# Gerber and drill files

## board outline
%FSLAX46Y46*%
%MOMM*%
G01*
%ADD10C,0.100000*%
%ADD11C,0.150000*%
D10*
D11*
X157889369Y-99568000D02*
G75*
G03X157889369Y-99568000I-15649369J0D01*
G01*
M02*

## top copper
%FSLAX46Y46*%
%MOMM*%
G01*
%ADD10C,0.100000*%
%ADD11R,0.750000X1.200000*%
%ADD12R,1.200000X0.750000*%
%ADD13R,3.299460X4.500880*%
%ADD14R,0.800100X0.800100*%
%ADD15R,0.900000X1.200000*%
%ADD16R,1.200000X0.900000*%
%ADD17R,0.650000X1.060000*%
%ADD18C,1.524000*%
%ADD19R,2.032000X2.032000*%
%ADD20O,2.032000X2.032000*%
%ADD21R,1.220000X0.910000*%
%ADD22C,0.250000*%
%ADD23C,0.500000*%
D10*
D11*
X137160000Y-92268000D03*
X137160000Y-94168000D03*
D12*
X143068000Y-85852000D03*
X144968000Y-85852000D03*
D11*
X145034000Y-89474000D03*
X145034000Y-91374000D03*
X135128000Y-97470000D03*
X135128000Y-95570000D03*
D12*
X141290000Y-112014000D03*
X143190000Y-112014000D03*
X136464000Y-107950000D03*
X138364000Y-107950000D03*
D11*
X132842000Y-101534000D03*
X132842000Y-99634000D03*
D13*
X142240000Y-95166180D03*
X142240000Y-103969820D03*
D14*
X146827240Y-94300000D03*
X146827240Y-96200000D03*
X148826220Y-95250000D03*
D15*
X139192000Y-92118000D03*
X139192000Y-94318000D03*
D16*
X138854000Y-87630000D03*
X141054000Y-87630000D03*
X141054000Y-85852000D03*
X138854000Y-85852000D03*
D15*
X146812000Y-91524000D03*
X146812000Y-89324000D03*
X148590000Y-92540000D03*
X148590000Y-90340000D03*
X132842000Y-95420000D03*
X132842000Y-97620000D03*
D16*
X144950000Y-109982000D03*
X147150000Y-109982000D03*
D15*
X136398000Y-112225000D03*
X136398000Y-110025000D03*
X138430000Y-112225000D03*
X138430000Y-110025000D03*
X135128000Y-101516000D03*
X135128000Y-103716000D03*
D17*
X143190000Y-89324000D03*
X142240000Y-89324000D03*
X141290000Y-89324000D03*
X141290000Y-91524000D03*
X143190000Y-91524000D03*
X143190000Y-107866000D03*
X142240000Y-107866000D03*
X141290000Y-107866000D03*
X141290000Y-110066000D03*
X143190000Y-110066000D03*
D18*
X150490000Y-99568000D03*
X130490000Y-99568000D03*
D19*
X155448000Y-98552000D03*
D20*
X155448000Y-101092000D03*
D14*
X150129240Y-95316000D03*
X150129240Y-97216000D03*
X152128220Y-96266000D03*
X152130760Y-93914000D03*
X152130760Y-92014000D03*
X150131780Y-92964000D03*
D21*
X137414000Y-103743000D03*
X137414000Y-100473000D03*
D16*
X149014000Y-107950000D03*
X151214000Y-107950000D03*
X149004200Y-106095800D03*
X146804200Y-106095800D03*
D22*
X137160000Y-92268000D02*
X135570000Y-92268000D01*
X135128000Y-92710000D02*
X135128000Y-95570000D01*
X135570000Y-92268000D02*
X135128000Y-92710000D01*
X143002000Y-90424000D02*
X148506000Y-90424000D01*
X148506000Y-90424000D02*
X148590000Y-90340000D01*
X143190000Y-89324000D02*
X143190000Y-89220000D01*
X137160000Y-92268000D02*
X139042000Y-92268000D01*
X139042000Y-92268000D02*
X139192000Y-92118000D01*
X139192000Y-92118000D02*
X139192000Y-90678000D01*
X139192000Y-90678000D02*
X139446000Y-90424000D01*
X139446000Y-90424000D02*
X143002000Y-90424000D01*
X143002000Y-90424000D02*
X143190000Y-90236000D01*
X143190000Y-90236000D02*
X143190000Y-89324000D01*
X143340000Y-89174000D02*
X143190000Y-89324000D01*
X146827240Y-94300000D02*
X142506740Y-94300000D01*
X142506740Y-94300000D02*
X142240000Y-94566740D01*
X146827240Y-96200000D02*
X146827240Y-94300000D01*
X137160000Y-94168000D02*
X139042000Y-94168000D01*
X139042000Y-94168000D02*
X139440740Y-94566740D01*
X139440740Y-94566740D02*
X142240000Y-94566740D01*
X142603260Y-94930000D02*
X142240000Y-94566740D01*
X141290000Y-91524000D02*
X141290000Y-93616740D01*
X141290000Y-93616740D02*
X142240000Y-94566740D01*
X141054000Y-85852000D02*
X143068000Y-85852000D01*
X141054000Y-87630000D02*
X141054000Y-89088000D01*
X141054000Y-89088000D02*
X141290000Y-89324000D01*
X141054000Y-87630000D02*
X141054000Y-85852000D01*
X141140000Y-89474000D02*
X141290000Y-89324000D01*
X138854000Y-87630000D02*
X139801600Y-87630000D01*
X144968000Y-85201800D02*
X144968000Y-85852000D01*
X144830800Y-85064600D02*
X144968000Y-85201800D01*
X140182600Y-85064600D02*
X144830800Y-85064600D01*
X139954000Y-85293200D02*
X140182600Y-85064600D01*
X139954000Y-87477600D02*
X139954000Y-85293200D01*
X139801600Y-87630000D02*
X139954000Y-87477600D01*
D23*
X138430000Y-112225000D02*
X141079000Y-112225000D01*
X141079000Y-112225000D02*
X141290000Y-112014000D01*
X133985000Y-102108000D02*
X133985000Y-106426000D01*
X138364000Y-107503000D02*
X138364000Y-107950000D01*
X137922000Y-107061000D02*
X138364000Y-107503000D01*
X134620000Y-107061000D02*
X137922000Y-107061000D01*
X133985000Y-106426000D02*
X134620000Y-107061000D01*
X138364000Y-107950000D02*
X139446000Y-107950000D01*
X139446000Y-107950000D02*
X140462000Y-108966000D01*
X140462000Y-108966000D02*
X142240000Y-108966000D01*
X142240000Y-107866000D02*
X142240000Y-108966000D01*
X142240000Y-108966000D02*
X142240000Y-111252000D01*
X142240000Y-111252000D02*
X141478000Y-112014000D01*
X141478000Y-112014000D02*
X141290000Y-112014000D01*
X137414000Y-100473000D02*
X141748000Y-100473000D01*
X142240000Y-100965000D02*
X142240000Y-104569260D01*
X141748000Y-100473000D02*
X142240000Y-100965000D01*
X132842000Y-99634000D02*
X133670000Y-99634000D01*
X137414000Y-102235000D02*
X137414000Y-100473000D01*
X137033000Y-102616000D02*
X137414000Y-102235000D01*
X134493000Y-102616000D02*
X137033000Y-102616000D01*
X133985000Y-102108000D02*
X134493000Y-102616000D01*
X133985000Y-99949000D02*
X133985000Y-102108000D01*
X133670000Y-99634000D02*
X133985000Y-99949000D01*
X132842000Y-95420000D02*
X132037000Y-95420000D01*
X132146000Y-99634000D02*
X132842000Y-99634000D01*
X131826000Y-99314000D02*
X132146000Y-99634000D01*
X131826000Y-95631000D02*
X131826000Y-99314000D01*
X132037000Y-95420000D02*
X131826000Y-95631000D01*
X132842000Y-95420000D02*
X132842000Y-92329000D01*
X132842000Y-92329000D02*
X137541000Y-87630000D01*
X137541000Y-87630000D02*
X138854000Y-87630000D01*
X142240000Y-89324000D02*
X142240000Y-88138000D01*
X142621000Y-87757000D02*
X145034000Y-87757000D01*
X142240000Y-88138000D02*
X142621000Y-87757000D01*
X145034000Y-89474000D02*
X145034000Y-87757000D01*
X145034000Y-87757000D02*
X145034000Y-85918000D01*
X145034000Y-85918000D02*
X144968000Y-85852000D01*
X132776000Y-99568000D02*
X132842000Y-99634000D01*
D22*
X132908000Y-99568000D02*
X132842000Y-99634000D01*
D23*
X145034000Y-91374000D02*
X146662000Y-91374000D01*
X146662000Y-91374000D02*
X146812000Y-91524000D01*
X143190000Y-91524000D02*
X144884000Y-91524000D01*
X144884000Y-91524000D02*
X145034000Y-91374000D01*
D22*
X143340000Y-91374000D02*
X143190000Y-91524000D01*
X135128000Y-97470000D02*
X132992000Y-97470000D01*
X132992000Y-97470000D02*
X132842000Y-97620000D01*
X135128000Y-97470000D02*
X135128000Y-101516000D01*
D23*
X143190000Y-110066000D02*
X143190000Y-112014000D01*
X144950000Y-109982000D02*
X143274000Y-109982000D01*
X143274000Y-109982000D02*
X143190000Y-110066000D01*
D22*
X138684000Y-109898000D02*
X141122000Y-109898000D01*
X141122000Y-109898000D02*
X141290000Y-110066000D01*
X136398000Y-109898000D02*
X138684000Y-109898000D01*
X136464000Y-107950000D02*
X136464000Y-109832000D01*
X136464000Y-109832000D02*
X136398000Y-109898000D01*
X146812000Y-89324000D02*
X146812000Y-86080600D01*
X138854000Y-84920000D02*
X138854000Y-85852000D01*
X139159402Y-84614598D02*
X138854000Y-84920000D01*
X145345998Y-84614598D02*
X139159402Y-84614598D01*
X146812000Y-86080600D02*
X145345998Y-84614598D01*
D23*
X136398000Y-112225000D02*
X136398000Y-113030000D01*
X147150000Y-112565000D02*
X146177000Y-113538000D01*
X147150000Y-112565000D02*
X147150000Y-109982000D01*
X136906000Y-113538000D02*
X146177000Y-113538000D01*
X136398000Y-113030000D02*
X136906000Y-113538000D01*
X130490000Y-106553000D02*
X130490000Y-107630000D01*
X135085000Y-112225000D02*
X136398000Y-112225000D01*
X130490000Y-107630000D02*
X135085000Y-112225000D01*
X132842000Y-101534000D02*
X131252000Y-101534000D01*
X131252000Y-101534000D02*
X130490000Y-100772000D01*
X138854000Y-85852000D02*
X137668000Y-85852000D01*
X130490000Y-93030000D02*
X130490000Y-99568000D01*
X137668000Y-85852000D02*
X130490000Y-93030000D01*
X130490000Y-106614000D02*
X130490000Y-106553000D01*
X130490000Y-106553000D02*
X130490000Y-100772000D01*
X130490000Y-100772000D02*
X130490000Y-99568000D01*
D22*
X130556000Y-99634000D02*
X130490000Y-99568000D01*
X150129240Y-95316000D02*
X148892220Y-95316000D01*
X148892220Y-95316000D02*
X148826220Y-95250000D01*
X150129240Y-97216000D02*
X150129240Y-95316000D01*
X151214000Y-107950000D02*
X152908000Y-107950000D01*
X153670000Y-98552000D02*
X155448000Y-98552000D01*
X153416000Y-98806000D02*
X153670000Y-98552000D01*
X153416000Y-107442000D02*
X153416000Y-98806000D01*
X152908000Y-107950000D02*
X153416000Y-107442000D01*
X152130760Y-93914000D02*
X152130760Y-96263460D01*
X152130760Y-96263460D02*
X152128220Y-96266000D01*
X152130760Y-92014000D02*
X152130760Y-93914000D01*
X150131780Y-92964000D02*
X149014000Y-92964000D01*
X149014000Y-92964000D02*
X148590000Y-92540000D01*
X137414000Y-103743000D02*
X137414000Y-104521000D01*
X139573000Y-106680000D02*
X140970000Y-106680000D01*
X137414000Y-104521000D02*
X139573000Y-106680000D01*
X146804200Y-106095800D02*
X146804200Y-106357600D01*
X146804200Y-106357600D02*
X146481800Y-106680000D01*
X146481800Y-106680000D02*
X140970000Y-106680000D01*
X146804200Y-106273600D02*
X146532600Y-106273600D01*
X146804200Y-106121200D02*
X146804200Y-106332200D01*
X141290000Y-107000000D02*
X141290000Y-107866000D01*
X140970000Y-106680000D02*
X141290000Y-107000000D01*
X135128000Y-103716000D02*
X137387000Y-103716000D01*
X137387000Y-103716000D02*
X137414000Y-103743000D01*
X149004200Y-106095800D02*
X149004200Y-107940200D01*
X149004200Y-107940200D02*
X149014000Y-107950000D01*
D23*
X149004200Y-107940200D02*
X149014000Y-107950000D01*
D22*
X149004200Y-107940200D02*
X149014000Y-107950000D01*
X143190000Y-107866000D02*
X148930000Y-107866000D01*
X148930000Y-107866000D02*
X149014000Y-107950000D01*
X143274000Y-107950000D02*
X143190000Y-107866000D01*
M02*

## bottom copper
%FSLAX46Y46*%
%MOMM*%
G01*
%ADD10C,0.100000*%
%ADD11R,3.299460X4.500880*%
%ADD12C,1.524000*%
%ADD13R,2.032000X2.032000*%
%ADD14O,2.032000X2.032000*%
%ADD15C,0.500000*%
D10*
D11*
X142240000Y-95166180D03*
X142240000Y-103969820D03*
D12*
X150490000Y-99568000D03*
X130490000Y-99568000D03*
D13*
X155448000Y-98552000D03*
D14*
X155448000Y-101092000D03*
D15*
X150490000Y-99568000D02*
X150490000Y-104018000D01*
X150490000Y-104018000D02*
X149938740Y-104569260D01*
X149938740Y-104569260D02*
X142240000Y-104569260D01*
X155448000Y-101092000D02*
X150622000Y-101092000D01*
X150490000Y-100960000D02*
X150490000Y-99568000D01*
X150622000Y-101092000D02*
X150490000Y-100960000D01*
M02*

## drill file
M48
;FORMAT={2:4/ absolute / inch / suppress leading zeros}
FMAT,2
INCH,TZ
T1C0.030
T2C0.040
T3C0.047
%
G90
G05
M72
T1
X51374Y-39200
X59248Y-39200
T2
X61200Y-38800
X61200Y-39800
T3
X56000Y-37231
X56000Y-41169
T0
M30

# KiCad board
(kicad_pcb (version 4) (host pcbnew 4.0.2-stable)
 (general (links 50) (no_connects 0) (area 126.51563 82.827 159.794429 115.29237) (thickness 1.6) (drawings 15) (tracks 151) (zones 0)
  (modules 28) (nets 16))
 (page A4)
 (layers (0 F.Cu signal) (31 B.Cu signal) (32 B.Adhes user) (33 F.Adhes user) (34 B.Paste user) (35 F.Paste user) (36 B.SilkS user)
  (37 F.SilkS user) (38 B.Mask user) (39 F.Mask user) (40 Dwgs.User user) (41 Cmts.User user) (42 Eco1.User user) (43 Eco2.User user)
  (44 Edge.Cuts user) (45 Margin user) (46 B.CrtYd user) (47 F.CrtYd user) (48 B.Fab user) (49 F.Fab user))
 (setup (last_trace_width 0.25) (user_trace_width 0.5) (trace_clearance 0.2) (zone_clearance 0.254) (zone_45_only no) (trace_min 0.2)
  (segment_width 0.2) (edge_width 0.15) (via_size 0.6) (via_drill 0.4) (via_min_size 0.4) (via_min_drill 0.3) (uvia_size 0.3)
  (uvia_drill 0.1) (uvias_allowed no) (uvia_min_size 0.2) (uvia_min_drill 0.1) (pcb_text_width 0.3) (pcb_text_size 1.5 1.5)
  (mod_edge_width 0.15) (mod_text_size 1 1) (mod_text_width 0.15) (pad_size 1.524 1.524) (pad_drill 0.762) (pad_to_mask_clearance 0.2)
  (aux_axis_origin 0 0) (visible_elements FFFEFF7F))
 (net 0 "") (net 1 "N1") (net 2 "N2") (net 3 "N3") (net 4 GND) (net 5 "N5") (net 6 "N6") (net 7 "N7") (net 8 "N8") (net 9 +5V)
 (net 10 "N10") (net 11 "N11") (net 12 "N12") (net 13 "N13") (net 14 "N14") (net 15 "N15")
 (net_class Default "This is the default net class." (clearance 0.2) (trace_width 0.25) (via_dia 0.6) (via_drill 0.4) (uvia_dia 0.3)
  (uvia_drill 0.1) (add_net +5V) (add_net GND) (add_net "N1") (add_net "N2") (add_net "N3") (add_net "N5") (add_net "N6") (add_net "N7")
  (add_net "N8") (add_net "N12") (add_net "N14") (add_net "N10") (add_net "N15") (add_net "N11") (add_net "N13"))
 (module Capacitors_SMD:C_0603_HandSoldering (layer F.Cu) (at 137.16 93.218 270)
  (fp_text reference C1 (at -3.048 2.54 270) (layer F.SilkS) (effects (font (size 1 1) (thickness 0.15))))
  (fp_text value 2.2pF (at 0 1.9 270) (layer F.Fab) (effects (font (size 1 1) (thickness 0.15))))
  (pad 1 smd rect (at -0.95 0 270) (size 1.2 0.75) (layers F.Cu F.Paste F.Mask) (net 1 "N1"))
  (pad 2 smd rect (at 0.95 0 270) (size 1.2 0.75) (layers F.Cu F.Paste F.Mask) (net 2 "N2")))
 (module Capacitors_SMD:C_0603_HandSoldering (layer F.Cu) (at 144.018 85.852)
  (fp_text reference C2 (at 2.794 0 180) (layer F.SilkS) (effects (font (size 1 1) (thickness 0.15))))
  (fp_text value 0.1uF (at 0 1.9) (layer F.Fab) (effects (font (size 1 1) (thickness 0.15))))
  (pad 1 smd rect (at -0.95 0) (size 1.2 0.75) (layers F.Cu F.Paste F.Mask) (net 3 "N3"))
  (pad 2 smd rect (at 0.95 0) (size 1.2 0.75) (layers F.Cu F.Paste F.Mask) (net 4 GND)))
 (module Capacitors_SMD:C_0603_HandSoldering (layer F.Cu) (at 145.034 90.424 270)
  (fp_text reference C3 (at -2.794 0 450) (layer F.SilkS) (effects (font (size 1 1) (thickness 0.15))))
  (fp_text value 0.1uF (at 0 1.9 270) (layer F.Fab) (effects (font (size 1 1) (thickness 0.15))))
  (pad 1 smd rect (at -0.95 0 270) (size 1.2 0.75) (layers F.Cu F.Paste F.Mask) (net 4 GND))
  (pad 2 smd rect (at 0.95 0 270) (size 1.2 0.75) (layers F.Cu F.Paste F.Mask) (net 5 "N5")))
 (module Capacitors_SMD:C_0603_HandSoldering (layer F.Cu) (at 135.128 96.52 90)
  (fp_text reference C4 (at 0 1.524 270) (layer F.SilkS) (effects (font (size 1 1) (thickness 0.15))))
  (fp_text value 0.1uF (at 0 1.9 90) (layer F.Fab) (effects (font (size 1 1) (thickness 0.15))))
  (pad 1 smd rect (at -0.95 0 90) (size 1.2 0.75) (layers F.Cu F.Paste F.Mask) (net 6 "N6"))
  (pad 2 smd rect (at 0.95 0 90) (size 1.2 0.75) (layers F.Cu F.Paste F.Mask) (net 1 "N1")))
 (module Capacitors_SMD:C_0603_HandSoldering (layer F.Cu) (at 142.24 112.014)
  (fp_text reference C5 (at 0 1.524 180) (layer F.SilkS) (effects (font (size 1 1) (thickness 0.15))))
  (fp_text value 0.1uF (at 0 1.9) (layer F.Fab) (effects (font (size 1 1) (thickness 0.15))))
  (pad 1 smd rect (at -0.95 0) (size 1.2 0.75) (layers F.Cu F.Paste F.Mask) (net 4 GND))
  (pad 2 smd rect (at 0.95 0) (size 1.2 0.75) (layers F.Cu F.Paste F.Mask) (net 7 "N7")))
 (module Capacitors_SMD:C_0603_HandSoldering (layer F.Cu) (at 137.414 107.95)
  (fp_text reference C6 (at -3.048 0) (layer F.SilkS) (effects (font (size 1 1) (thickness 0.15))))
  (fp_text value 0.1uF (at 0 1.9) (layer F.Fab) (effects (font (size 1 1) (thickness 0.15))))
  (pad 1 smd rect (at -0.95 0) (size 1.2 0.75) (layers F.Cu F.Paste F.Mask) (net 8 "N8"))
  (pad 2 smd rect (at 0.95 0) (size 1.2 0.75) (layers F.Cu F.Paste F.Mask) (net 4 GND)))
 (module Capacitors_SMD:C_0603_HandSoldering (layer F.Cu) (at 132.842 100.584 90)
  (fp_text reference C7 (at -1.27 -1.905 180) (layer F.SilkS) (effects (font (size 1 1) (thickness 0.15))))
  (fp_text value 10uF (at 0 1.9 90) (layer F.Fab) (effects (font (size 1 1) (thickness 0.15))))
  (pad 1 smd rect (at -0.95 0 90) (size 1.2 0.75) (layers F.Cu F.Paste F.Mask) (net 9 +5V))
  (pad 2 smd rect (at 0.95 0 90) (size 1.2 0.75) (layers F.Cu F.Paste F.Mask) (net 4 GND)))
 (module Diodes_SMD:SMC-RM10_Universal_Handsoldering (layer F.Cu) (at 142.24 99.568 270)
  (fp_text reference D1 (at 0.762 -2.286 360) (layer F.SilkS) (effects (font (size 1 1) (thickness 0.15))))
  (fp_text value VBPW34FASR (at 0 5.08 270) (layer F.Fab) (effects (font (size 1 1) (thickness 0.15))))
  (pad 1 thru_hole rect (at -5.00126 0 270) (size 4.50088 3.29946) (drill 1.19888 (offset 0.59944 0)) (layers *.Cu *.Mask F.SilkS)
   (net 2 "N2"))
  (pad 2 thru_hole rect (at 5.00126 0 90) (size 4.50088 3.29946) (drill 1.19888 (offset 0.59944 0)) (layers *.Cu *.Mask F.SilkS) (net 4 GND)))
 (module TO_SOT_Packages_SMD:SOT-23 (layer F.Cu) (at 147.828 95.25 270)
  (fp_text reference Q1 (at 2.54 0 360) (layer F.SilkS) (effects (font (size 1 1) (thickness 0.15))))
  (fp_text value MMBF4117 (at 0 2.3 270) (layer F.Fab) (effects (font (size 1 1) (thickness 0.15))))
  (pad 1 smd rect (at -0.95 1.00076 270) (size 0.8001 0.8001) (layers F.Cu F.Paste F.Mask) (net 2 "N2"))
  (pad 2 smd rect (at 0.95 1.00076 270) (size 0.8001 0.8001) (layers F.Cu F.Paste F.Mask) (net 2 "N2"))
  (pad 3 smd rect (at 0 -0.99822 270) (size 0.8001 0.8001) (layers F.Cu F.Paste F.Mask) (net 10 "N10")))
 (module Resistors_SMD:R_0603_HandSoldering (layer F.Cu) (at 139.192 93.218 270)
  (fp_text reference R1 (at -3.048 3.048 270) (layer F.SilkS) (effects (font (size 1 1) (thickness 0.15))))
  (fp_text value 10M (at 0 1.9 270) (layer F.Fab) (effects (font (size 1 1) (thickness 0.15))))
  (pad 1 smd rect (at -1.1 0 270) (size 1.2 0.9) (layers F.Cu F.Paste F.Mask) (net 1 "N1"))
  (pad 2 smd rect (at 1.1 0 270) (size 1.2 0.9) (layers F.Cu F.Paste F.Mask) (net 2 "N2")))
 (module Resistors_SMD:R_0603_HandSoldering (layer F.Cu) (at 139.954 87.63)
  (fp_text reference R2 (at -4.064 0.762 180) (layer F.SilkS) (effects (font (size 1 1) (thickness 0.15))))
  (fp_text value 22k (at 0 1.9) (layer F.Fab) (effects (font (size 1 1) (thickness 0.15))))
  (pad 1 smd rect (at -1.1 0) (size 1.2 0.9) (layers F.Cu F.Paste F.Mask) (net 4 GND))
  (pad 2 smd rect (at 1.1 0) (size 1.2 0.9) (layers F.Cu F.Paste F.Mask) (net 3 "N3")))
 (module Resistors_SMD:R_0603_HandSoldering (layer F.Cu) (at 139.954 85.852 180)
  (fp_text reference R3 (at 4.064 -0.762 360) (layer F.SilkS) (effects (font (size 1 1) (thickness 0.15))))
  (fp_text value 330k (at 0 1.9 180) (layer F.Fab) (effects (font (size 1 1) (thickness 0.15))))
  (pad 1 smd rect (at -1.1 0 180) (size 1.2 0.9) (layers F.Cu F.Paste F.Mask) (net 3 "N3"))
  (pad 2 smd rect (at 1.1 0 180) (size 1.2 0.9) (layers F.Cu F.Paste F.Mask) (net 9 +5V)))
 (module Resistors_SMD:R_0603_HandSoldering (layer F.Cu) (at 146.812 90.424 90)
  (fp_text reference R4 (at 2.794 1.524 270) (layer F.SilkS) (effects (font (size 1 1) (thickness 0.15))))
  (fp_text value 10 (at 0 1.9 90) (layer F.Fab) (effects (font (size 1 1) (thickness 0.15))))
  (pad 1 smd rect (at -1.1 0 90) (size 1.2 0.9) (layers F.Cu F.Paste F.Mask) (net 5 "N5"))
  (pad 2 smd rect (at 1.1 0 90) (size 1.2 0.9) (layers F.Cu F.Paste F.Mask) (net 9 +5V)))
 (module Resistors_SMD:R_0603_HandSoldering (layer F.Cu) (at 148.59 91.44 90)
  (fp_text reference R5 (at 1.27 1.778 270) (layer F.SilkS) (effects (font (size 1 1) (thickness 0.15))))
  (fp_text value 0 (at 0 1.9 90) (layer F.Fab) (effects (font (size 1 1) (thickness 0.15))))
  (pad 1 smd rect (at -1.1 0 90) (size 1.2 0.9) (layers F.Cu F.Paste F.Mask) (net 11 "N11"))
  (pad 2 smd rect (at 1.1 0 90) (size 1.2 0.9) (layers F.Cu F.Paste F.Mask) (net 1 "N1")))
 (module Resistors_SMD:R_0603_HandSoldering (layer F.Cu) (at 132.842 96.52 270)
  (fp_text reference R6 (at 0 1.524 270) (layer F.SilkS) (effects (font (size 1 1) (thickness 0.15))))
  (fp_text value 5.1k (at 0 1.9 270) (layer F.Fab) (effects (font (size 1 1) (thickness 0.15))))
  (pad 1 smd rect (at -1.1 0 270) (size 1.2 0.9) (layers F.Cu F.Paste F.Mask) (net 4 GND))
  (pad 2 smd rect (at 1.1 0 270) (size 1.2 0.9) (layers F.Cu F.Paste F.Mask) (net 6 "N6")))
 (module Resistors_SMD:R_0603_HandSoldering (layer F.Cu) (at 146.05 109.982)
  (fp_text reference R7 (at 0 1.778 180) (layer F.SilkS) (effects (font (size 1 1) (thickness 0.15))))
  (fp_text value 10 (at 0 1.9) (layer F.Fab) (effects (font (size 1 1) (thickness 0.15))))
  (pad 1 smd rect (at -1.1 0) (size 1.2 0.9) (layers F.Cu F.Paste F.Mask) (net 7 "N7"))
  (pad 2 smd rect (at 1.1 0) (size 1.2 0.9) (layers F.Cu F.Paste F.Mask) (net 9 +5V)))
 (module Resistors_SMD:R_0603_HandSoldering (layer F.Cu) (at 136.398 111.125 90)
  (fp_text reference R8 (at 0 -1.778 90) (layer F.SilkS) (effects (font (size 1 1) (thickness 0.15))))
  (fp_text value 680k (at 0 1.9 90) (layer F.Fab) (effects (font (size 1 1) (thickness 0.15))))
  (pad 1 smd rect (at -1.1 0 90) (size 1.2 0.9) (layers F.Cu F.Paste F.Mask) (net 9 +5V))
  (pad 2 smd rect (at 1.1 0 90) (size 1.2 0.9) (layers F.Cu F.Paste F.Mask) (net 8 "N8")))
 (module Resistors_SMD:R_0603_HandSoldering (layer F.Cu) (at 138.43 111.125 90)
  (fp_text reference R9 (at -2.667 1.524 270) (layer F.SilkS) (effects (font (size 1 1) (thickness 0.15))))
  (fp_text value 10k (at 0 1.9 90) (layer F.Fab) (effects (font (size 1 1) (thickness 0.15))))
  (pad 1 smd rect (at -1.1 0 90) (size 1.2 0.9) (layers F.Cu F.Paste F.Mask) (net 4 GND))
  (pad 2 smd rect (at 1.1 0 90) (size 1.2 0.9) (layers F.Cu F.Paste F.Mask) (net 8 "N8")))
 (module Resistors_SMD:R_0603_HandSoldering (layer F.Cu) (at 135.128 102.616 270)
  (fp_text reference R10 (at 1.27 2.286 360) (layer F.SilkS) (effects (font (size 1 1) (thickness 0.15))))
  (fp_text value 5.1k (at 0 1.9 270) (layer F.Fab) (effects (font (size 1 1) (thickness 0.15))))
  (pad 1 smd rect (at -1.1 0 270) (size 1.2 0.9) (layers F.Cu F.Paste F.Mask) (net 6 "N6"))
  (pad 2 smd rect (at 1.1 0 270) (size 1.2 0.9) (layers F.Cu F.Paste F.Mask) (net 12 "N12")))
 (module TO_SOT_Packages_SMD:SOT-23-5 (layer F.Cu) (at 142.24 90.424 270)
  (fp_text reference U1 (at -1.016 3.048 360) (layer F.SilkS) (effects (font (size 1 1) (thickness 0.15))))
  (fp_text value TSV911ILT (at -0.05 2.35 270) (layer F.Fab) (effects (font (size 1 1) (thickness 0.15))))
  (pad 1 smd rect (at -1.1 -0.95 270) (size 1.06 0.65) (layers F.Cu F.Paste F.Mask) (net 1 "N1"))
  (pad 2 smd rect (at -1.1 0 270) (size 1.06 0.65) (layers F.Cu F.Paste F.Mask) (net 4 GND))
  (pad 3 smd rect (at -1.1 0.95 270) (size 1.06 0.65) (layers F.Cu F.Paste F.Mask) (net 3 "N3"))
  (pad 4 smd rect (at 1.1 0.95 270) (size 1.06 0.65) (layers F.Cu F.Paste F.Mask) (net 2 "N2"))
  (pad 5 smd rect (at 1.1 -0.95 270) (size 1.06 0.65) (layers F.Cu F.Paste F.Mask) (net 5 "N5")))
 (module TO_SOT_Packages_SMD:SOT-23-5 (layer F.Cu) (at 142.24 108.966 270)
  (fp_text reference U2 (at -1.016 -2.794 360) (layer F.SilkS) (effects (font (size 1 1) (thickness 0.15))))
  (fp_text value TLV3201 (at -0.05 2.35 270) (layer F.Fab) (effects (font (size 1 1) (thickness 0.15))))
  (pad 1 smd rect (at -1.1 -0.95 270) (size 1.06 0.65) (layers F.Cu F.Paste F.Mask) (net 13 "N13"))
  (pad 2 smd rect (at -1.1 0 270) (size 1.06 0.65) (layers F.Cu F.Paste F.Mask) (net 4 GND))
  (pad 3 smd rect (at -1.1 0.95 270) (size 1.06 0.65) (layers F.Cu F.Paste F.Mask) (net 12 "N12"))
  (pad 4 smd rect (at 1.1 0.95 270) (size 1.06 0.65) (layers F.Cu F.Paste F.Mask) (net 8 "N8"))
  (pad 5 smd rect (at 1.1 -0.95 270) (size 1.06 0.65) (layers F.Cu F.Paste F.Mask) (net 7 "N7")))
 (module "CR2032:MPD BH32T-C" (layer B.Cu) (at 142.24 99.568 90)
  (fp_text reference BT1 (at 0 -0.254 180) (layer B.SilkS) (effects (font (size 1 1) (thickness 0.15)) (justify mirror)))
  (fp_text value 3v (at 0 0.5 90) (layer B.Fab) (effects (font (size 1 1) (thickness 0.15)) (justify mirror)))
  (pad 2 thru_hole circle (at 0 8.25 90) (size 1.524 1.524) (drill 0.762) (layers *.Cu *.Mask B.SilkS) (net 4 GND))
  (pad 1 thru_hole circle (at 0 -11.75 90) (size 1.524 1.524) (drill 0.762) (layers *.Cu *.Mask B.SilkS) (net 9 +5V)))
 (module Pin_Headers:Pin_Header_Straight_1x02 (layer F.Cu) (at 155.448 98.552)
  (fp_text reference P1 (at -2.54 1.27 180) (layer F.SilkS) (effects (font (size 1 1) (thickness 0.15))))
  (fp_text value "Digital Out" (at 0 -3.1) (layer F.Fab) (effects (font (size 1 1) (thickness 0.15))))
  (pad 1 thru_hole rect (at 0 0) (size 2.032 2.032) (drill 1.016) (layers *.Cu *.Mask F.SilkS) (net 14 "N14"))
  (pad 2 thru_hole oval (at 0 2.54) (size 2.032 2.032) (drill 1.016) (layers *.Cu *.Mask F.SilkS) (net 4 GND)))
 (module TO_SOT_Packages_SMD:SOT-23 (layer F.Cu) (at 151.13 96.266 270)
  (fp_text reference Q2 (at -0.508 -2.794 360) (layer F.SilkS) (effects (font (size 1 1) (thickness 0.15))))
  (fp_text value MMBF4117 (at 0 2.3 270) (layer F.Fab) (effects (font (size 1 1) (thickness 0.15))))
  (pad 1 smd rect (at -0.95 1.00076 270) (size 0.8001 0.8001) (layers F.Cu F.Paste F.Mask) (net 10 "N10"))
  (pad 2 smd rect (at 0.95 1.00076 270) (size 0.8001 0.8001) (layers F.Cu F.Paste F.Mask) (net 10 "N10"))
  (pad 3 smd rect (at 0 -0.99822 270) (size 0.8001 0.8001) (layers F.Cu F.Paste F.Mask) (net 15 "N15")))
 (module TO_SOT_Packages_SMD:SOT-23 (layer F.Cu) (at 151.13 92.964 90)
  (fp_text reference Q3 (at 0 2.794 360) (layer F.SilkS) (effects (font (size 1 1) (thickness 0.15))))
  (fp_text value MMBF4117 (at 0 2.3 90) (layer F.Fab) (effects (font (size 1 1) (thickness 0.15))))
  (pad 1 smd rect (at -0.95 1.00076 90) (size 0.8001 0.8001) (layers F.Cu F.Paste F.Mask) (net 15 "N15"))
  (pad 2 smd rect (at 0.95 1.00076 90) (size 0.8001 0.8001) (layers F.Cu F.Paste F.Mask) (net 15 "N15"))
  (pad 3 smd rect (at 0 -0.99822 90) (size 0.8001 0.8001) (layers F.Cu F.Paste F.Mask) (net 11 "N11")))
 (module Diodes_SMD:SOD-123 (layer F.Cu) (at 137.414 102.108 90)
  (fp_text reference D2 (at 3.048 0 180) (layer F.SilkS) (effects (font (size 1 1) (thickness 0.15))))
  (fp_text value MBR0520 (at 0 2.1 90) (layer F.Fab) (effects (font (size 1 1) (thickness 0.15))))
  (pad 1 smd rect (at -1.635 0 90) (size 0.91 1.22) (layers F.Cu F.Paste F.Mask) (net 12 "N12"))
  (pad 2 smd rect (at 1.635 0 90) (size 0.91 1.22) (layers F.Cu F.Paste F.Mask) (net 4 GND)))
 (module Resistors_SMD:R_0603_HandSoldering (layer F.Cu) (at 150.114 107.95)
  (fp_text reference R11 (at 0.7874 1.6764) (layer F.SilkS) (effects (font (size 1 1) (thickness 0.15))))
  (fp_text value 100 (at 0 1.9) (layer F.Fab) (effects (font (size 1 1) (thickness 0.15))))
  (pad 1 smd rect (at -1.1 0) (size 1.2 0.9) (layers F.Cu F.Paste F.Mask) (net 13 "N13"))
  (pad 2 smd rect (at 1.1 0) (size 1.2 0.9) (layers F.Cu F.Paste F.Mask) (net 14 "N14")))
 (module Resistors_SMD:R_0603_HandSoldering (layer F.Cu) (at 147.9042 106.0958 180)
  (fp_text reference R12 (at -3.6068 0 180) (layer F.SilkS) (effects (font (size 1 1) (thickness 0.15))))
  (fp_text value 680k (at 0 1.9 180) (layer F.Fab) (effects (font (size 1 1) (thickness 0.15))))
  (pad 1 smd rect (at -1.1 0 180) (size 1.2 0.9) (layers F.Cu F.Paste F.Mask) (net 13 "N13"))
  (pad 2 smd rect (at 1.1 0 180) (size 1.2 0.9) (layers F.Cu F.Paste F.Mask) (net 12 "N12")))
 (gr_circle (center 142.24 99.568) (end 154.94 108.712) (layer Edge.Cuts) (width 0.15))
 (segment (start 137.16 92.268) (end 135.57 92.268) (width 0.25) (layer F.Cu) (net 1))
 (segment (start 135.128 92.71) (end 135.128 95.57) (width 0.25) (layer F.Cu) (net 1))
 (segment (start 135.57 92.268) (end 135.128 92.71) (width 0.25) (layer F.Cu) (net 1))
 (segment (start 143.002 90.424) (end 148.506 90.424) (width 0.25) (layer F.Cu) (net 1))
 (segment (start 148.506 90.424) (end 148.59 90.34) (width 0.25) (layer F.Cu) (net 1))
 (segment (start 143.19 89.324) (end 143.19 89.22) (width 0.25) (layer F.Cu) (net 1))
 (segment (start 137.16 92.268) (end 139.042 92.268) (width 0.25) (layer F.Cu) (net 1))
 (segment (start 139.042 92.268) (end 139.192 92.118) (width 0.25) (layer F.Cu) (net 1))
 (segment (start 139.192 92.118) (end 139.192 90.678) (width 0.25) (layer F.Cu) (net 1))
 (segment (start 139.192 90.678) (end 139.446 90.424) (width 0.25) (layer F.Cu) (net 1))
 (segment (start 139.446 90.424) (end 143.002 90.424) (width 0.25) (layer F.Cu) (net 1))
 (segment (start 143.002 90.424) (end 143.19 90.236) (width 0.25) (layer F.Cu) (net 1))
 (segment (start 143.19 90.236) (end 143.19 89.324) (width 0.25) (layer F.Cu) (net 1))
 (segment (start 143.34 89.174) (end 143.19 89.324) (width 0.25) (layer F.Cu) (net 1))
 (segment (start 146.82724 94.3) (end 142.50674 94.3) (width 0.25) (layer F.Cu) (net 2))
 (segment (start 142.50674 94.3) (end 142.24 94.56674) (width 0.25) (layer F.Cu) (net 2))
 (segment (start 146.82724 96.2) (end 146.82724 94.3) (width 0.25) (layer F.Cu) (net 2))
 (segment (start 137.16 94.168) (end 139.042 94.168) (width 0.25) (layer F.Cu) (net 2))
 (segment (start 139.042 94.168) (end 139.44074 94.56674) (width 0.25) (layer F.Cu) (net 2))
 (segment (start 139.44074 94.56674) (end 142.24 94.56674) (width 0.25) (layer F.Cu) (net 2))
 (segment (start 142.60326 94.93) (end 142.24 94.56674) (width 0.25) (layer F.Cu) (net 2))
 (segment (start 141.29 91.524) (end 141.29 93.61674) (width 0.25) (layer F.Cu) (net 2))
 (segment (start 141.29 93.61674) (end 142.24 94.56674) (width 0.25) (layer F.Cu) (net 2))
 (segment (start 141.054 85.852) (end 143.068 85.852) (width 0.25) (layer F.Cu) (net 3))
 (segment (start 141.054 87.63) (end 141.054 89.088) (width 0.25) (layer F.Cu) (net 3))
 (segment (start 141.054 89.088) (end 141.29 89.324) (width 0.25) (layer F.Cu) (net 3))
 (segment (start 141.054 87.63) (end 141.054 85.852) (width 0.25) (layer F.Cu) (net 3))
 (segment (start 141.14 89.474) (end 141.29 89.324) (width 0.25) (layer F.Cu) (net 3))
 (segment (start 138.854 87.63) (end 139.8016 87.63) (width 0.25) (layer F.Cu) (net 4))
 (segment (start 144.968 85.2018) (end 144.968 85.852) (width 0.25) (layer F.Cu) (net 4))
 (segment (start 144.8308 85.0646) (end 144.968 85.2018) (width 0.25) (layer F.Cu) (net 4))
 (segment (start 140.1826 85.0646) (end 144.8308 85.0646) (width 0.25) (layer F.Cu) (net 4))
 (segment (start 139.954 85.2932) (end 140.1826 85.0646) (width 0.25) (layer F.Cu) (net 4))
 (segment (start 139.954 87.4776) (end 139.954 85.2932) (width 0.25) (layer F.Cu) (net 4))
 (segment (start 139.8016 87.63) (end 139.954 87.4776) (width 0.25) (layer F.Cu) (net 4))
 (segment (start 138.43 112.225) (end 141.079 112.225) (width 0.5) (layer F.Cu) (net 4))
 (segment (start 141.079 112.225) (end 141.29 112.014) (width 0.5) (layer F.Cu) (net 4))
 (segment (start 133.985 102.108) (end 133.985 106.426) (width 0.5) (layer F.Cu) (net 4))
 (segment (start 138.364 107.503) (end 138.364 107.95) (width 0.5) (layer F.Cu) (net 4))
 (segment (start 137.922 107.061) (end 138.364 107.503) (width 0.5) (layer F.Cu) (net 4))
 (segment (start 134.62 107.061) (end 137.922 107.061) (width 0.5) (layer F.Cu) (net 4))
 (segment (start 133.985 106.426) (end 134.62 107.061) (width 0.5) (layer F.Cu) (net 4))
 (segment (start 138.364 107.95) (end 139.446 107.95) (width 0.5) (layer F.Cu) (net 4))
 (segment (start 139.446 107.95) (end 140.462 108.966) (width 0.5) (layer F.Cu) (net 4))
 (segment (start 140.462 108.966) (end 142.24 108.966) (width 0.5) (layer F.Cu) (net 4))
 (segment (start 142.24 107.866) (end 142.24 108.966) (width 0.5) (layer F.Cu) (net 4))
 (segment (start 142.24 108.966) (end 142.24 111.252) (width 0.5) (layer F.Cu) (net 4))
 (segment (start 142.24 111.252) (end 141.478 112.014) (width 0.5) (layer F.Cu) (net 4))
 (segment (start 141.478 112.014) (end 141.29 112.014) (width 0.5) (layer F.Cu) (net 4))
 (segment (start 137.414 100.473) (end 141.748 100.473) (width 0.5) (layer F.Cu) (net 4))
 (segment (start 142.24 100.965) (end 142.24 104.56926) (width 0.5) (layer F.Cu) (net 4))
 (segment (start 141.748 100.473) (end 142.24 100.965) (width 0.5) (layer F.Cu) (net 4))
 (segment (start 132.842 99.634) (end 133.67 99.634) (width 0.5) (layer F.Cu) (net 4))
 (segment (start 137.414 102.235) (end 137.414 100.473) (width 0.5) (layer F.Cu) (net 4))
 (segment (start 137.033 102.616) (end 137.414 102.235) (width 0.5) (layer F.Cu) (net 4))
 (segment (start 134.493 102.616) (end 137.033 102.616) (width 0.5) (layer F.Cu) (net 4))
 (segment (start 133.985 102.108) (end 134.493 102.616) (width 0.5) (layer F.Cu) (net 4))
 (segment (start 133.985 99.949) (end 133.985 102.108) (width 0.5) (layer F.Cu) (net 4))
 (segment (start 133.67 99.634) (end 133.985 99.949) (width 0.5) (layer F.Cu) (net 4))
 (segment (start 132.842 95.42) (end 132.037 95.42) (width 0.5) (layer F.Cu) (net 4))
 (segment (start 132.146 99.634) (end 132.842 99.634) (width 0.5) (layer F.Cu) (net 4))
 (segment (start 131.826 99.314) (end 132.146 99.634) (width 0.5) (layer F.Cu) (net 4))
 (segment (start 131.826 95.631) (end 131.826 99.314) (width 0.5) (layer F.Cu) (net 4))
 (segment (start 132.037 95.42) (end 131.826 95.631) (width 0.5) (layer F.Cu) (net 4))
 (segment (start 132.842 95.42) (end 132.842 92.329) (width 0.5) (layer F.Cu) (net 4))
 (segment (start 132.842 92.329) (end 137.541 87.63) (width 0.5) (layer F.Cu) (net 4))
 (segment (start 137.541 87.63) (end 138.854 87.63) (width 0.5) (layer F.Cu) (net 4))
 (segment (start 142.24 89.324) (end 142.24 88.138) (width 0.5) (layer F.Cu) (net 4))
 (segment (start 142.621 87.757) (end 145.034 87.757) (width 0.5) (layer F.Cu) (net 4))
 (segment (start 142.24 88.138) (end 142.621 87.757) (width 0.5) (layer F.Cu) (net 4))
 (segment (start 145.034 89.474) (end 145.034 87.757) (width 0.5) (layer F.Cu) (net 4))
 (segment (start 145.034 87.757) (end 145.034 85.918) (width 0.5) (layer F.Cu) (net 4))
 (segment (start 145.034 85.918) (end 144.968 85.852) (width 0.5) (layer F.Cu) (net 4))
 (segment (start 150.49 99.568) (end 150.49 104.018) (width 0.5) (layer B.Cu) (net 4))
 (segment (start 150.49 104.018) (end 149.93874 104.56926) (width 0.5) (layer B.Cu) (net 4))
 (segment (start 149.93874 104.56926) (end 142.24 104.56926) (width 0.5) (layer B.Cu) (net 4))
 (segment (start 155.448 101.092) (end 150.622 101.092) (width 0.5) (layer B.Cu) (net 4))
 (segment (start 150.49 100.96) (end 150.49 99.568) (width 0.5) (layer B.Cu) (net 4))
 (segment (start 150.622 101.092) (end 150.49 100.96) (width 0.5) (layer B.Cu) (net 4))
 (segment (start 132.776 99.568) (end 132.842 99.634) (width 0.5) (layer F.Cu) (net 4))
 (segment (start 132.908 99.568) (end 132.842 99.634) (width 0.25) (layer F.Cu) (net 4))
 (segment (start 145.034 91.374) (end 146.662 91.374) (width 0.5) (layer F.Cu) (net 5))
 (segment (start 146.662 91.374) (end 146.812 91.524) (width 0.5) (layer F.Cu) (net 5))
 (segment (start 143.19 91.524) (end 144.884 91.524) (width 0.5) (layer F.Cu) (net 5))
 (segment (start 144.884 91.524) (end 145.034 91.374) (width 0.5) (layer F.Cu) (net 5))
 (segment (start 143.34 91.374) (end 143.19 91.524) (width 0.25) (layer F.Cu) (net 5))
 (segment (start 135.128 97.47) (end 132.992 97.47) (width 0.25) (layer F.Cu) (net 6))
 (segment (start 132.992 97.47) (end 132.842 97.62) (width 0.25) (layer F.Cu) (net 6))
 (segment (start 135.128 97.47) (end 135.128 101.516) (width 0.25) (layer F.Cu) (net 6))
 (segment (start 143.19 110.066) (end 143.19 112.014) (width 0.5) (layer F.Cu) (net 7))
 (segment (start 144.95 109.982) (end 143.274 109.982) (width 0.5) (layer F.Cu) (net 7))
 (segment (start 143.274 109.982) (end 143.19 110.066) (width 0.5) (layer F.Cu) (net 7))
 (segment (start 138.684 109.898) (end 141.122 109.898) (width 0.25) (layer F.Cu) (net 8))
 (segment (start 141.122 109.898) (end 141.29 110.066) (width 0.25) (layer F.Cu) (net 8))
 (segment (start 136.398 109.898) (end 138.684 109.898) (width 0.25) (layer F.Cu) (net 8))
 (segment (start 136.464 107.95) (end 136.464 109.832) (width 0.25) (layer F.Cu) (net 8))
 (segment (start 136.464 109.832) (end 136.398 109.898) (width 0.25) (layer F.Cu) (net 8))
 (segment (start 146.812 89.324) (end 146.812 86.0806) (width 0.25) (layer F.Cu) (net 9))
 (segment (start 138.854 84.92) (end 138.854 85.852) (width 0.25) (layer F.Cu) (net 9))
 (segment (start 139.159402 84.614598) (end 138.854 84.92) (width 0.25) (layer F.Cu) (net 9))
 (segment (start 145.345998 84.614598) (end 139.159402 84.614598) (width 0.25) (layer F.Cu) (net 9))
 (segment (start 146.812 86.0806) (end 145.345998 84.614598) (width 0.25) (layer F.Cu) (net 9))
 (segment (start 136.398 112.225) (end 136.398 113.03) (width 0.5) (layer F.Cu) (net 9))
 (segment (start 147.15 112.565) (end 146.177 113.538) (width 0.5) (layer F.Cu) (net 9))
 (segment (start 147.15 112.565) (end 147.15 109.982) (width 0.5) (layer F.Cu) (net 9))
 (segment (start 136.906 113.538) (end 146.177 113.538) (width 0.5) (layer F.Cu) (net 9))
 (segment (start 136.398 113.03) (end 136.906 113.538) (width 0.5) (layer F.Cu) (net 9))
 (segment (start 130.49 106.553) (end 130.49 107.63) (width 0.5) (layer F.Cu) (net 9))
 (segment (start 135.085 112.225) (end 136.398 112.225) (width 0.5) (layer F.Cu) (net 9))
 (segment (start 130.49 107.63) (end 135.085 112.225) (width 0.5) (layer F.Cu) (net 9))
 (segment (start 132.842 101.534) (end 131.252 101.534) (width 0.5) (layer F.Cu) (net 9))
 (segment (start 131.252 101.534) (end 130.49 100.772) (width 0.5) (layer F.Cu) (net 9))
 (segment (start 138.854 85.852) (end 137.668 85.852) (width 0.5) (layer F.Cu) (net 9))
 (segment (start 130.49 93.03) (end 130.49 99.568) (width 0.5) (layer F.Cu) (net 9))
 (segment (start 137.668 85.852) (end 130.49 93.03) (width 0.5) (layer F.Cu) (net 9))
 (segment (start 130.49 106.614) (end 130.49 106.553) (width 0.5) (layer F.Cu) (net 9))
 (segment (start 130.49 106.553) (end 130.49 100.772) (width 0.5) (layer F.Cu) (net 9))
 (segment (start 130.49 100.772) (end 130.49 99.568) (width 0.5) (layer F.Cu) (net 9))
 (segment (start 130.556 99.634) (end 130.49 99.568) (width 0.25) (layer F.Cu) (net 9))
 (segment (start 150.12924 95.316) (end 148.89222 95.316) (width 0.25) (layer F.Cu) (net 10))
 (segment (start 148.89222 95.316) (end 148.82622 95.25) (width 0.25) (layer F.Cu) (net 10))
 (segment (start 150.12924 97.216) (end 150.12924 95.316) (width 0.25) (layer F.Cu) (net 10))
 (segment (start 151.214 107.95) (end 152.908 107.95) (width 0.25) (layer F.Cu) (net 14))
 (segment (start 153.67 98.552) (end 155.448 98.552) (width 0.25) (layer F.Cu) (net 14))
 (segment (start 153.416 98.806) (end 153.67 98.552) (width 0.25) (layer F.Cu) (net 14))
 (segment (start 153.416 107.442) (end 153.416 98.806) (width 0.25) (layer F.Cu) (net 14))
 (segment (start 152.908 107.95) (end 153.416 107.442) (width 0.25) (layer F.Cu) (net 14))
 (segment (start 152.13076 93.914) (end 152.13076 96.26346) (width 0.25) (layer F.Cu) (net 15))
 (segment (start 152.13076 96.26346) (end 152.12822 96.266) (width 0.25) (layer F.Cu) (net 15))
 (segment (start 152.13076 92.014) (end 152.13076 93.914) (width 0.25) (layer F.Cu) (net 15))
 (segment (start 150.13178 92.964) (end 149.014 92.964) (width 0.25) (layer F.Cu) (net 11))
 (segment (start 149.014 92.964) (end 148.59 92.54) (width 0.25) (layer F.Cu) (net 11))
 (segment (start 137.414 103.743) (end 137.414 104.521) (width 0.25) (layer F.Cu) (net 12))
 (segment (start 139.573 106.68) (end 140.97 106.68) (width 0.25) (layer F.Cu) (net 12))
 (segment (start 137.414 104.521) (end 139.573 106.68) (width 0.25) (layer F.Cu) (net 12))
 (segment (start 146.8042 106.0958) (end 146.8042 106.3576) (width 0.25) (layer F.Cu) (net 12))
 (segment (start 146.8042 106.3576) (end 146.4818 106.68) (width 0.25) (layer F.Cu) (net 12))
 (segment (start 146.4818 106.68) (end 140.97 106.68) (width 0.25) (layer F.Cu) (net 12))
 (segment (start 146.8042 106.2736) (end 146.5326 106.2736) (width 0.25) (layer F.Cu) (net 12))
 (segment (start 146.8042 106.1212) (end 146.8042 106.3322) (width 0.25) (layer F.Cu) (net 12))
 (segment (start 141.29 107) (end 141.29 107.866) (width 0.25) (layer F.Cu) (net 12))
 (segment (start 140.97 106.68) (end 141.29 107) (width 0.25) (layer F.Cu) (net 12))
 (segment (start 135.128 103.716) (end 137.387 103.716) (width 0.25) (layer F.Cu) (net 12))
 (segment (start 137.387 103.716) (end 137.414 103.743) (width 0.25) (layer F.Cu) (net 12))
 (segment (start 149.0042 106.0958) (end 149.0042 107.9402) (width 0.25) (layer F.Cu) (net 13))
 (segment (start 149.0042 107.9402) (end 149.014 107.95) (width 0.25) (layer F.Cu) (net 13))
 (segment (start 149.0042 107.9402) (end 149.014 107.95) (width 0.5) (layer F.Cu) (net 13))
 (segment (start 149.0042 107.9402) (end 149.014 107.95) (width 0.25) (layer F.Cu) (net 13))
 (segment (start 143.19 107.866) (end 148.93 107.866) (width 0.25) (layer F.Cu) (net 13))
 (segment (start 148.93 107.866) (end 149.014 107.95) (width 0.25) (layer F.Cu) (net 13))
 (segment (start 143.274 107.95) (end 143.19 107.866) (width 0.25) (layer F.Cu) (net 13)))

